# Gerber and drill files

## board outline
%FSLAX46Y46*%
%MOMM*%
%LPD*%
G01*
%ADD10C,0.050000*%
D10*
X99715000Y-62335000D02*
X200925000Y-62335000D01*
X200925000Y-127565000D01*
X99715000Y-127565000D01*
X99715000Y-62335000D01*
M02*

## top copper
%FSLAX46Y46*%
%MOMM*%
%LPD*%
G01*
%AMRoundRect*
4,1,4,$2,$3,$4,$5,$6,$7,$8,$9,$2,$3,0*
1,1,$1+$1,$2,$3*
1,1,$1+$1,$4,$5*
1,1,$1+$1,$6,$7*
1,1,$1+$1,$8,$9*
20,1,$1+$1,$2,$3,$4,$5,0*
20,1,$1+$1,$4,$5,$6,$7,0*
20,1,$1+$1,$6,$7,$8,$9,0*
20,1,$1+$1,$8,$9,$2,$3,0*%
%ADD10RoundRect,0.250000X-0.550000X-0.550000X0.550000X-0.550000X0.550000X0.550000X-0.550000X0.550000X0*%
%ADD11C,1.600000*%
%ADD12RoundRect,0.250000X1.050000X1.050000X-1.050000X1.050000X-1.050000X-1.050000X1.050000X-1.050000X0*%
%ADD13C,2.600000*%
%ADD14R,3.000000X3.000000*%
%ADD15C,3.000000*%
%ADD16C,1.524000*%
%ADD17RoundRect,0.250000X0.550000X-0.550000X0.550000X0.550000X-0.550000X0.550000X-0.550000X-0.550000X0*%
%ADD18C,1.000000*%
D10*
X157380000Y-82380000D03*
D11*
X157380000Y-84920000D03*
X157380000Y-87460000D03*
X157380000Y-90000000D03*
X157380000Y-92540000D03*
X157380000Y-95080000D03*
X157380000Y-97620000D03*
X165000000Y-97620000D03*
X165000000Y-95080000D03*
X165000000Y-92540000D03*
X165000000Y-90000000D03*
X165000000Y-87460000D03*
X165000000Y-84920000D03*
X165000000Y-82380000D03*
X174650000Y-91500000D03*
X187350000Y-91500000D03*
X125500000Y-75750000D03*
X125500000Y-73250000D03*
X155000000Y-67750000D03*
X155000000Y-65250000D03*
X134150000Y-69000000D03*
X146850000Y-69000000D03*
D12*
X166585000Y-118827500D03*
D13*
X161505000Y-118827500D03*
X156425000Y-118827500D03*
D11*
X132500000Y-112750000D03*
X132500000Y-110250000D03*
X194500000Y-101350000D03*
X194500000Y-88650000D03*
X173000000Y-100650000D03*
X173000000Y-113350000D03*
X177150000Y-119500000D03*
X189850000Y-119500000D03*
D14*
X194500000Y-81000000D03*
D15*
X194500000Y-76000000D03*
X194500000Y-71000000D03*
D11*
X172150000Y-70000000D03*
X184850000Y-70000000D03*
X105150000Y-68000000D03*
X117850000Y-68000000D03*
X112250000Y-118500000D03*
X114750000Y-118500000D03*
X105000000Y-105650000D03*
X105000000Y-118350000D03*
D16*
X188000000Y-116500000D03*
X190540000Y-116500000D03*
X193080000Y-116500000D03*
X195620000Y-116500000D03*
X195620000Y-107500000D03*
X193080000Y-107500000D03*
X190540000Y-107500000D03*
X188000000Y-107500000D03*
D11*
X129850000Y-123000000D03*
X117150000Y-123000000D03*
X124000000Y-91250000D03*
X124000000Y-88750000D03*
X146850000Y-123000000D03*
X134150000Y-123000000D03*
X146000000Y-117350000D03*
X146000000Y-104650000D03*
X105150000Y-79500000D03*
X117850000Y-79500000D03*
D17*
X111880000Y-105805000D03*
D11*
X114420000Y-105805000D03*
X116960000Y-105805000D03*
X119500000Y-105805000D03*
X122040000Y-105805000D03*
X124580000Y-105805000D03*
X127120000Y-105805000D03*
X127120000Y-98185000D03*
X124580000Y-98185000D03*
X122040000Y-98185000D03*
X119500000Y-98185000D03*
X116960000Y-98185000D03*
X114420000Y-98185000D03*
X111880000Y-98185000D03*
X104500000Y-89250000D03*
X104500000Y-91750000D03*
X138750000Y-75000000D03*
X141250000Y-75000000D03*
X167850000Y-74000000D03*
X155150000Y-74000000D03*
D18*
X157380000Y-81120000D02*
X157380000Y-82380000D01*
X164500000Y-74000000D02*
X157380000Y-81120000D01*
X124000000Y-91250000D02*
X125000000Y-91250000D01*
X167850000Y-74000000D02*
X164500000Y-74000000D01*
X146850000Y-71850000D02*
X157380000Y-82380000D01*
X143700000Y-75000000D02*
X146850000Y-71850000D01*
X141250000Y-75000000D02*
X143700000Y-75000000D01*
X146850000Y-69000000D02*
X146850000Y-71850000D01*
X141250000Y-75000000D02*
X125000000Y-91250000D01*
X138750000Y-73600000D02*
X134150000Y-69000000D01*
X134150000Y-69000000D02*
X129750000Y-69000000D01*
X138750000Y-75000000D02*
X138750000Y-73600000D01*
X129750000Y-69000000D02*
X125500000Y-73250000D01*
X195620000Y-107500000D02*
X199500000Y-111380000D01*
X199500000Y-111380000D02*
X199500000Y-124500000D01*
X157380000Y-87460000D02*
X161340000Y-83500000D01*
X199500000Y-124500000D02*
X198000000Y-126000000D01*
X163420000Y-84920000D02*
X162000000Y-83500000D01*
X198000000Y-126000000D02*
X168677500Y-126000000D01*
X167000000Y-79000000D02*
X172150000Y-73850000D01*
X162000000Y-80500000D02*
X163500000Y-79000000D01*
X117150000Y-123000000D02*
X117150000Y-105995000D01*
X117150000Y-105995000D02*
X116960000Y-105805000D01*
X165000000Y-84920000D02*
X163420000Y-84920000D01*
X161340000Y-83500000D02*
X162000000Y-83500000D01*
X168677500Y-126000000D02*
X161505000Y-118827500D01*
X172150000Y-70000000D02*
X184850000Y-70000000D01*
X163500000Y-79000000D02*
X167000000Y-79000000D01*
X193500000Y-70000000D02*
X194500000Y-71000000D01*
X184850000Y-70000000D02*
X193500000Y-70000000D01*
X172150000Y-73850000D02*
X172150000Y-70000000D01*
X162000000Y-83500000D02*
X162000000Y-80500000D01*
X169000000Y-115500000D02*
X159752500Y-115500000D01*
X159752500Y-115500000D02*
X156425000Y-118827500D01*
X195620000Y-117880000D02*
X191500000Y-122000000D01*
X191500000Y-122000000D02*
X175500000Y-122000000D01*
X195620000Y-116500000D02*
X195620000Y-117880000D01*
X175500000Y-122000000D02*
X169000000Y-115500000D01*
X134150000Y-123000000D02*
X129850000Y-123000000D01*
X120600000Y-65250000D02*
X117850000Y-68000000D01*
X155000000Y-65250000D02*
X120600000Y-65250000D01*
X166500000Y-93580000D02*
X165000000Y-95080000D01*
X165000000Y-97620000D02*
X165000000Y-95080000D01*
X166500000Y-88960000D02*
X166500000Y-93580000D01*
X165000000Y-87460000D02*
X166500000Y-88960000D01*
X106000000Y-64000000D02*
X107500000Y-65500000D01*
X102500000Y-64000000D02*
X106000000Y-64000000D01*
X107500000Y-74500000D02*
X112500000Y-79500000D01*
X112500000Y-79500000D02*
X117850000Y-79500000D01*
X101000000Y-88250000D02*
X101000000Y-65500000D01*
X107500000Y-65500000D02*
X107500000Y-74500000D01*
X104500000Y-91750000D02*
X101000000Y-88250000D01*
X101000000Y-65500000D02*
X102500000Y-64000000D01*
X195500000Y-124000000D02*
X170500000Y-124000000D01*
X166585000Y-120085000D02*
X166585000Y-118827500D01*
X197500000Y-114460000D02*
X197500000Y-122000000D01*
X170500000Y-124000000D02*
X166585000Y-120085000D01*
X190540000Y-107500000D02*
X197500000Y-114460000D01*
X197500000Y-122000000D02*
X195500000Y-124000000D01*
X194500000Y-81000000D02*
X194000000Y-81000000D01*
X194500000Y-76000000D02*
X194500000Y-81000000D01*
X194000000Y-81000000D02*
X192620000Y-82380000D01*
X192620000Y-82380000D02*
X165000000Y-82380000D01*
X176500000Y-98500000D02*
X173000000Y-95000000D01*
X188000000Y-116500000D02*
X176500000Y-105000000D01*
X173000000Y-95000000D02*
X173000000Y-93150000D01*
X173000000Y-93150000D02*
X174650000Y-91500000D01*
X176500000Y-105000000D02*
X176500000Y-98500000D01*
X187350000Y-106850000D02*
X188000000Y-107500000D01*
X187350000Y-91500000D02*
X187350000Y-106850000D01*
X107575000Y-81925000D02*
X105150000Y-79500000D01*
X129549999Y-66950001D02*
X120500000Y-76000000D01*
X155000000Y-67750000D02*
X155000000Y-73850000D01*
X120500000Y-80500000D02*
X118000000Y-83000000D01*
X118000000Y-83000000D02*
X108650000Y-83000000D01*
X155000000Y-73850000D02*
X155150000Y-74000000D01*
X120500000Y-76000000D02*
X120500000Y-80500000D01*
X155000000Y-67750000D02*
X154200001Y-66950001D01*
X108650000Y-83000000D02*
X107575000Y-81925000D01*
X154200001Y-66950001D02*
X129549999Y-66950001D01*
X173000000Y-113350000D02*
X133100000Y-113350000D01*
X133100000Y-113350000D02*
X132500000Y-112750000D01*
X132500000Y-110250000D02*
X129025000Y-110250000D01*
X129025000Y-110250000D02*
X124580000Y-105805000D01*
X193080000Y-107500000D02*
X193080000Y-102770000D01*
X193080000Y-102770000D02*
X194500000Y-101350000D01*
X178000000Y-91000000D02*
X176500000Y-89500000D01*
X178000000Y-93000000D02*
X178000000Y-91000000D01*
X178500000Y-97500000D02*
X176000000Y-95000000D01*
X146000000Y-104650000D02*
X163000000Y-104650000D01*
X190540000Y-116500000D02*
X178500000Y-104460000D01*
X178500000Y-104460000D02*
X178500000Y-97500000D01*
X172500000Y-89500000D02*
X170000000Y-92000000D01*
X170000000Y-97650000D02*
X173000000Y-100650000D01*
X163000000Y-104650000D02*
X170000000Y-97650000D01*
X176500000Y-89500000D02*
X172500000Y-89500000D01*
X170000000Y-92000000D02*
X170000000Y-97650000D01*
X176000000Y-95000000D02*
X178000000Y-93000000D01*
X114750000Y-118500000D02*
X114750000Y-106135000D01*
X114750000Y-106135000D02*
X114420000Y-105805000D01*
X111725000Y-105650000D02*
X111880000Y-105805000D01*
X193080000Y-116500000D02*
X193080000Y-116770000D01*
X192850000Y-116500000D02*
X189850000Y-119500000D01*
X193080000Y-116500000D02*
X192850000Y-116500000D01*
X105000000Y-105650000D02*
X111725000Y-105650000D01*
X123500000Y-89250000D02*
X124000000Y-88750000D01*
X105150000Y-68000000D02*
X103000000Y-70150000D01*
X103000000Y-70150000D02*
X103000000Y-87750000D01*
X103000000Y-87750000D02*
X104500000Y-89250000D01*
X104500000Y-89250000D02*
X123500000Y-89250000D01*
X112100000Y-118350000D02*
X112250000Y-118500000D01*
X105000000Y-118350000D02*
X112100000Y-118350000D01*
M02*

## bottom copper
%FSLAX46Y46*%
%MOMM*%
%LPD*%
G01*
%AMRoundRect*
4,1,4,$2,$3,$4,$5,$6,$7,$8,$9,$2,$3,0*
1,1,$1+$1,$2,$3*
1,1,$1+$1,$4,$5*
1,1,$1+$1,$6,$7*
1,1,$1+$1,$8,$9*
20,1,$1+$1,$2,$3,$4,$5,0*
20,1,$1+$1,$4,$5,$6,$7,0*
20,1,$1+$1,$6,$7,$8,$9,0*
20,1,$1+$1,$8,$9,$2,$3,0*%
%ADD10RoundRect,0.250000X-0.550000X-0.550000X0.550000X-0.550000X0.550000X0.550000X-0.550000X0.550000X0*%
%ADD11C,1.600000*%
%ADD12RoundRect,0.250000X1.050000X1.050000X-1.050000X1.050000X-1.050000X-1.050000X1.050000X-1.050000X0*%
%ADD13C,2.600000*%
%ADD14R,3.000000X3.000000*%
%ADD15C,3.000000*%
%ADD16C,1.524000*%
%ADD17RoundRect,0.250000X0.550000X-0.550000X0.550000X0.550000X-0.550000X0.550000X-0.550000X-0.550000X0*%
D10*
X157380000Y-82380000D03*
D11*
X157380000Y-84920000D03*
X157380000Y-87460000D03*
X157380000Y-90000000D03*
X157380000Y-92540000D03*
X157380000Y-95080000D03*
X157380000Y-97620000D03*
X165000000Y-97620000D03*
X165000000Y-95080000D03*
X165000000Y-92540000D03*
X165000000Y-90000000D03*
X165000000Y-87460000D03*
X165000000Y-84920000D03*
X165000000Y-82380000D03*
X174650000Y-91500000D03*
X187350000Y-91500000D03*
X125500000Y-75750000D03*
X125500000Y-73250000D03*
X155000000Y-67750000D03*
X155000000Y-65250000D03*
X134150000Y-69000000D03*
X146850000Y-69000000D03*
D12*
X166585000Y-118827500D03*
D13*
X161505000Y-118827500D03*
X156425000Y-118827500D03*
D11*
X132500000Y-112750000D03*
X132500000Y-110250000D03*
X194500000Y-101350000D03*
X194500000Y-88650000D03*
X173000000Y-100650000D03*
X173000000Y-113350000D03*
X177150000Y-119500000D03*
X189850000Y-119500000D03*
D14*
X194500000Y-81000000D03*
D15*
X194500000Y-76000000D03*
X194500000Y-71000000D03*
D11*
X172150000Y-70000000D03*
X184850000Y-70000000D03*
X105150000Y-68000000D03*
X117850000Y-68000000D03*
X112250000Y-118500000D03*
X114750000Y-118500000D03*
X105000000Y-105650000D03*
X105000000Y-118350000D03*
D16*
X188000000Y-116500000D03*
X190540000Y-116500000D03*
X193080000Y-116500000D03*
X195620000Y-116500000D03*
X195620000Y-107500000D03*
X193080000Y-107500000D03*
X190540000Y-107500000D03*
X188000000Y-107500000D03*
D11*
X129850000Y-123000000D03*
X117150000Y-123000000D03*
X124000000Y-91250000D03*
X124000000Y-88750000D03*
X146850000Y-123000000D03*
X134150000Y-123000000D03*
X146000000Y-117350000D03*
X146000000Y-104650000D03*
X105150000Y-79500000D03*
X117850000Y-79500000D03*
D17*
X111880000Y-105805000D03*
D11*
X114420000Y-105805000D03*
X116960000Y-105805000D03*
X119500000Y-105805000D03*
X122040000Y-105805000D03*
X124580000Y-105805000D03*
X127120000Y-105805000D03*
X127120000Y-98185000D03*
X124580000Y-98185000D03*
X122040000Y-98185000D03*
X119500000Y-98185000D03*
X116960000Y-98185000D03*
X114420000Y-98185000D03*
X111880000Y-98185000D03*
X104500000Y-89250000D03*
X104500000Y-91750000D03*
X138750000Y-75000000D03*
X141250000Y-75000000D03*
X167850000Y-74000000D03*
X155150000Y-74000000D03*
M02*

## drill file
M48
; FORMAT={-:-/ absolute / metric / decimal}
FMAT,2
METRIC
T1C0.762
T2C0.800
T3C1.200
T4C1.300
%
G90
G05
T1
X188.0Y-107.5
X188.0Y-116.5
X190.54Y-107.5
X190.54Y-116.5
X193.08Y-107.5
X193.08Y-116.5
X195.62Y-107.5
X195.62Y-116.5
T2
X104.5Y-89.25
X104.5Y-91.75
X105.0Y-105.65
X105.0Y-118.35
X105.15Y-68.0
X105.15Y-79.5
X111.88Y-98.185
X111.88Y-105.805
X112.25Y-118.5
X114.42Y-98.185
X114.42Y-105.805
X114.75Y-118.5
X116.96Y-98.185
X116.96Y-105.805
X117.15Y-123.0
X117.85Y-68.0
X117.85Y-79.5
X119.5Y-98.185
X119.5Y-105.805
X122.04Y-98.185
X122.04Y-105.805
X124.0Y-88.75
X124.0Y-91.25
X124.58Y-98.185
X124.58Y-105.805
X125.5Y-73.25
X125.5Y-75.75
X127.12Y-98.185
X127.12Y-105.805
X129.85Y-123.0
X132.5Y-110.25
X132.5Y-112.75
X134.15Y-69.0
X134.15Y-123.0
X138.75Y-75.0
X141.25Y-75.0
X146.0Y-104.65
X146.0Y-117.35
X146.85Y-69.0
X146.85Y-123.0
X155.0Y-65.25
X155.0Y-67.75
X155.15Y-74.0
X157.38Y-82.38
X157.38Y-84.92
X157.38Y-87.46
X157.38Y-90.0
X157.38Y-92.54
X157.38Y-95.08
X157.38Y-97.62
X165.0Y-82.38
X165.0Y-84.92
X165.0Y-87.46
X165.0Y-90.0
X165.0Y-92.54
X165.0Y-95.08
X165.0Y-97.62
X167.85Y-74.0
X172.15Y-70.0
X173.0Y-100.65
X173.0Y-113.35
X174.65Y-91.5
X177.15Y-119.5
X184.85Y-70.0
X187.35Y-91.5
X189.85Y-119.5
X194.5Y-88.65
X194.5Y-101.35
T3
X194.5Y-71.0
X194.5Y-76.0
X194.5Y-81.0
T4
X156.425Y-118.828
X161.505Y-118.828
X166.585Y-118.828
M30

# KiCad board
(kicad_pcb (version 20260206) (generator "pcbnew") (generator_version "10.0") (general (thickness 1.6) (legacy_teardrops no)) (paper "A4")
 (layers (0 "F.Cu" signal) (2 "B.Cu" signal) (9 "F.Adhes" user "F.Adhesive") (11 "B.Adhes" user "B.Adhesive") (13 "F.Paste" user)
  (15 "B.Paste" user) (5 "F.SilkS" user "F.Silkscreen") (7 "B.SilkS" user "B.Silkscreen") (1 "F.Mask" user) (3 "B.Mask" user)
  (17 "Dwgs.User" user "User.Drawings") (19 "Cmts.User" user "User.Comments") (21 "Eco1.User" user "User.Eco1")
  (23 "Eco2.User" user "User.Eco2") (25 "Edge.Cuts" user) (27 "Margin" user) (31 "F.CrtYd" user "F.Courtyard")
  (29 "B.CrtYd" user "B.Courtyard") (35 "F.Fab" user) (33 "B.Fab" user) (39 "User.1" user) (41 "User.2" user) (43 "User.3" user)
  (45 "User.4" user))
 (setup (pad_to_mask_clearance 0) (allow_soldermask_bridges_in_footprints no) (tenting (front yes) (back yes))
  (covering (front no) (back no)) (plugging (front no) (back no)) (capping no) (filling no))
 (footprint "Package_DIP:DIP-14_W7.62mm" (layer "F.Cu") (at 157.38 82.38)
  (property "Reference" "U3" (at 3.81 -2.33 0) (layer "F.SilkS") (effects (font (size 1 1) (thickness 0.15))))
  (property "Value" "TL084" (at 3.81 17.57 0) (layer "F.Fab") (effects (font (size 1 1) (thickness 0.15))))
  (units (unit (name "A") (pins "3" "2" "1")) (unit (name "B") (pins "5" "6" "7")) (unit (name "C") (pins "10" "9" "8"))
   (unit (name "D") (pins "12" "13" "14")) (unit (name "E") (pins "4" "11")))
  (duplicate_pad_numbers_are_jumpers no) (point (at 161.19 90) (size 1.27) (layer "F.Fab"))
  (pad "1" thru_hole roundrect (at 0 0) (size 1.6 1.6) (drill 0.8) (layers "*.Cu" "*.Mask") (remove_unused_layers no)
   (roundrect_rratio 0.15625) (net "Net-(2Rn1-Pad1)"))
  (pad "2" thru_hole circle (at 0 2.54) (size 1.6 1.6) (drill 0.8) (layers "*.Cu" "*.Mask") (remove_unused_layers no) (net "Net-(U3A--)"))
  (pad "3" thru_hole circle (at 0 5.08) (size 1.6 1.6) (drill 0.8) (layers "*.Cu" "*.Mask") (remove_unused_layers no) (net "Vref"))
  (pad "4" thru_hole circle (at 0 7.62) (size 1.6 1.6) (drill 0.8) (layers "*.Cu" "*.Mask") (remove_unused_layers no) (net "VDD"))
  (pad "5" thru_hole circle (at 0 10.16) (size 1.6 1.6) (drill 0.8) (layers "*.Cu" "*.Mask") (remove_unused_layers no) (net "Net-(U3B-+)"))
  (pad "6" thru_hole circle (at 0 12.7) (size 1.6 1.6) (drill 0.8) (layers "*.Cu" "*.Mask") (remove_unused_layers no) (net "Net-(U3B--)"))
  (pad "7" thru_hole circle (at 0 15.24) (size 1.6 1.6) (drill 0.8) (layers "*.Cu" "*.Mask") (remove_unused_layers no) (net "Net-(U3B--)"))
  (pad "8" thru_hole circle (at 7.62 15.24) (size 1.6 1.6) (drill 0.8) (layers "*.Cu" "*.Mask") (remove_unused_layers no)
   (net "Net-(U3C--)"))
  (pad "9" thru_hole circle (at 7.62 12.7) (size 1.6 1.6) (drill 0.8) (layers "*.Cu" "*.Mask") (remove_unused_layers no) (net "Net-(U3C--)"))
  (pad "10" thru_hole circle (at 7.62 10.16) (size 1.6 1.6) (drill 0.8) (layers "*.Cu" "*.Mask") (remove_unused_layers no)
   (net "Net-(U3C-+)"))
  (pad "11" thru_hole circle (at 7.62 7.62) (size 1.6 1.6) (drill 0.8) (layers "*.Cu" "*.Mask") (remove_unused_layers no) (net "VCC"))
  (pad "12" thru_hole circle (at 7.62 5.08) (size 1.6 1.6) (drill 0.8) (layers "*.Cu" "*.Mask") (remove_unused_layers no)
   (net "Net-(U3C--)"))
  (pad "13" thru_hole circle (at 7.62 2.54) (size 1.6 1.6) (drill 0.8) (layers "*.Cu" "*.Mask") (remove_unused_layers no) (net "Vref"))
  (pad "14" thru_hole circle (at 7.62 0) (size 1.6 1.6) (drill 0.8) (layers "*.Cu" "*.Mask") (remove_unused_layers no) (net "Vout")))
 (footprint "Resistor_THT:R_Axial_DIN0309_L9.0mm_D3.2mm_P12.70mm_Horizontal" (layer "F.Cu") (at 174.65 91.5)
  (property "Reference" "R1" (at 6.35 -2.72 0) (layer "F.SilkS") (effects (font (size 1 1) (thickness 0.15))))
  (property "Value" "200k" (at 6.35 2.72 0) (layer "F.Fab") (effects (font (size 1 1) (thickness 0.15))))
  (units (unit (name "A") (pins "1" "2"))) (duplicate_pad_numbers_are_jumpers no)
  (pad "1" thru_hole circle (at 0 0) (size 1.6 1.6) (drill 0.8) (layers "*.Cu" "*.Mask") (remove_unused_layers no) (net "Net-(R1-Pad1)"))
  (pad "2" thru_hole circle (at 12.7 0) (size 1.6 1.6) (drill 0.8) (layers "*.Cu" "*.Mask") (remove_unused_layers no) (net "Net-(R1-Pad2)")))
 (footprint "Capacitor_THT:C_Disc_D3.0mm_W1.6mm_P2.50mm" (layer "F.Cu") (at 125.5 75.75 90)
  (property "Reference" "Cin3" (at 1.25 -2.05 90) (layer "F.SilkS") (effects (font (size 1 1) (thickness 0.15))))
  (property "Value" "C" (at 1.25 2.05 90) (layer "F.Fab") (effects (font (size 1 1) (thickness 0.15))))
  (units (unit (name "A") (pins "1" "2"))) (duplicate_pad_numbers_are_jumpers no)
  (pad "1" thru_hole circle (at 0 0 90) (size 1.6 1.6) (drill 0.8) (layers "*.Cu" "*.Mask") (remove_unused_layers no)
   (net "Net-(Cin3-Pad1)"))
  (pad "2" thru_hole circle (at 2.5 0 90) (size 1.6 1.6) (drill 0.8) (layers "*.Cu" "*.Mask") (remove_unused_layers no) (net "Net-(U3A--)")))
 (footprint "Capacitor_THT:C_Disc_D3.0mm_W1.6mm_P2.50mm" (layer "F.Cu") (at 155 67.75 90)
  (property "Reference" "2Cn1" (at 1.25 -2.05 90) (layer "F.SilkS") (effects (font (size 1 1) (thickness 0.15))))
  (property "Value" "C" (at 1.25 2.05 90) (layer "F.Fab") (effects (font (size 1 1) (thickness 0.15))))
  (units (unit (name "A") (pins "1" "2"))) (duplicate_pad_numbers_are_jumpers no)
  (pad "1" thru_hole circle (at 0 0 90) (size 1.6 1.6) (drill 0.8) (layers "*.Cu" "*.Mask") (remove_unused_layers no)
   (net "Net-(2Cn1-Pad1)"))
  (pad "2" thru_hole circle (at 2.5 0 90) (size 1.6 1.6) (drill 0.8) (layers "*.Cu" "*.Mask") (remove_unused_layers no) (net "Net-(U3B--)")))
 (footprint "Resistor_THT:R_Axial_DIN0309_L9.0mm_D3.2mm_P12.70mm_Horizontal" (layer "F.Cu") (at 134.15 69)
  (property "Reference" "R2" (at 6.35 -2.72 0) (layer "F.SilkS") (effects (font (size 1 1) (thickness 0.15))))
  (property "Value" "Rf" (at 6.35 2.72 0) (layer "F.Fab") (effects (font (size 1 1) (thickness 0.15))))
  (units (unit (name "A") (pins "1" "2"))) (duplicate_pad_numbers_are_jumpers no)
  (pad "1" thru_hole circle (at 0 0) (size 1.6 1.6) (drill 0.8) (layers "*.Cu" "*.Mask") (remove_unused_layers no) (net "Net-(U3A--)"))
  (pad "2" thru_hole circle (at 12.7 0) (size 1.6 1.6) (drill 0.8) (layers "*.Cu" "*.Mask") (remove_unused_layers no)
   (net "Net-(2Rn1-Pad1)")))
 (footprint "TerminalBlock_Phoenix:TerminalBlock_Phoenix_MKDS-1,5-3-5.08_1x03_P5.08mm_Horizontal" (layer "F.Cu") (at 166.585 118.8275 180)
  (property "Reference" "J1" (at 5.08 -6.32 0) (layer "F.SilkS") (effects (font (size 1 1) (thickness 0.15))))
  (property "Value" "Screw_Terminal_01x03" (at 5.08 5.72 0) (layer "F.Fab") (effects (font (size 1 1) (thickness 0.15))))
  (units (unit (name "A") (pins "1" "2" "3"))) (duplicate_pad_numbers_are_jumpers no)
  (pad "1" thru_hole roundrect (at 0 0 180) (size 2.6 2.6) (drill 1.3) (layers "*.Cu" "*.Mask") (remove_unused_layers no)
   (roundrect_rratio 0.096154) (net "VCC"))
  (pad "2" thru_hole circle (at 5.08 0 180) (size 2.6 2.6) (drill 1.3) (layers "*.Cu" "*.Mask") (remove_unused_layers no) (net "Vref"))
  (pad "3" thru_hole circle (at 10.16 0 180) (size 2.6 2.6) (drill 1.3) (layers "*.Cu" "*.Mask") (remove_unused_layers no) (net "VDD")))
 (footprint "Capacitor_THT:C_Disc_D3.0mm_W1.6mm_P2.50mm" (layer "F.Cu") (at 132.5 112.75 90)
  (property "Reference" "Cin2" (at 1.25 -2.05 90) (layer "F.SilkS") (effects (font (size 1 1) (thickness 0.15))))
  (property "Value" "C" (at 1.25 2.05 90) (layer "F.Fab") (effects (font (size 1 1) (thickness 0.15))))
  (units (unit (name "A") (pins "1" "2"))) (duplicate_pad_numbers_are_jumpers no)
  (pad "1" thru_hole circle (at 0 0 90) (size 1.6 1.6) (drill 0.8) (layers "*.Cu" "*.Mask") (remove_unused_layers no)
   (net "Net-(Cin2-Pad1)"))
  (pad "2" thru_hole circle (at 2.5 0 90) (size 1.6 1.6) (drill 0.8) (layers "*.Cu" "*.Mask") (remove_unused_layers no) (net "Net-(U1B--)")))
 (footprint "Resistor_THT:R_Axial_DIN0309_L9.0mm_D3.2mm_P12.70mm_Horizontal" (layer "F.Cu") (at 194.5 101.35 90)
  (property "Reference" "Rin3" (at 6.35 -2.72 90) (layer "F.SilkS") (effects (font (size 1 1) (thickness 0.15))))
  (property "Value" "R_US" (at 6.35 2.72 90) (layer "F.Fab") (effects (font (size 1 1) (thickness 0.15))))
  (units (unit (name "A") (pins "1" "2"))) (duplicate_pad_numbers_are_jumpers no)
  (pad "1" thru_hole circle (at 0 0 90) (size 1.6 1.6) (drill 0.8) (layers "*.Cu" "*.Mask") (remove_unused_layers no) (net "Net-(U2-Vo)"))
  (pad "2" thru_hole circle (at 12.7 0 90) (size 1.6 1.6) (drill 0.8) (layers "*.Cu" "*.Mask") (remove_unused_layers no)
   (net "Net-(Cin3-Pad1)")))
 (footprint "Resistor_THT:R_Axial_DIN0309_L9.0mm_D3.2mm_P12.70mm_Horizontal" (layer "F.Cu") (at 173 100.65 -90)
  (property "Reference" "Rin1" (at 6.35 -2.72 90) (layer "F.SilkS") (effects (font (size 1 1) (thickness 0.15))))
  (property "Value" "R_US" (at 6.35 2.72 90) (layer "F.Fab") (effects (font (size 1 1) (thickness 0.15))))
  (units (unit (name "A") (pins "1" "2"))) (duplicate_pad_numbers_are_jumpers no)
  (pad "1" thru_hole circle (at 0 0 270) (size 1.6 1.6) (drill 0.8) (layers "*.Cu" "*.Mask") (remove_unused_layers no) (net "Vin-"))
  (pad "2" thru_hole circle (at 12.7 0 270) (size 1.6 1.6) (drill 0.8) (layers "*.Cu" "*.Mask") (remove_unused_layers no)
   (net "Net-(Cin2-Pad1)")))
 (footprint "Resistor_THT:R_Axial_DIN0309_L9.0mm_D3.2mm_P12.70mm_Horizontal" (layer "F.Cu") (at 177.15 119.5)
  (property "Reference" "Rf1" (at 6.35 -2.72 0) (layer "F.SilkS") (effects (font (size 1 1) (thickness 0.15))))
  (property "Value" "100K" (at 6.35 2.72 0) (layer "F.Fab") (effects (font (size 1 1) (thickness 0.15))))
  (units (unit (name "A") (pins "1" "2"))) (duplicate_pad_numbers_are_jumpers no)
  (pad "1" thru_hole circle (at 0 0) (size 1.6 1.6) (drill 0.8) (layers "*.Cu" "*.Mask") (remove_unused_layers no) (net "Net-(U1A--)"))
  (pad "2" thru_hole circle (at 12.7 0) (size 1.6 1.6) (drill 0.8) (layers "*.Cu" "*.Mask") (remove_unused_layers no) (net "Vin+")))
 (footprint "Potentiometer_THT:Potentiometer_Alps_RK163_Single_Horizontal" (layer "F.Cu") (at 194.5 81 180)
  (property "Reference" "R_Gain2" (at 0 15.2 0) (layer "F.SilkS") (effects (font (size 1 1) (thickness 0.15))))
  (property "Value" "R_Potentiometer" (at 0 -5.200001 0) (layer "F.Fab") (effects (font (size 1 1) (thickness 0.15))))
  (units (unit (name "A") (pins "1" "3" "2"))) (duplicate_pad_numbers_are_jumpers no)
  (pad "1" thru_hole rect (at 0 0) (size 3 3) (drill 1.2) (layers "*.Cu" "*.Mask") (remove_unused_layers no) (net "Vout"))
  (pad "2" thru_hole circle (at 0 5) (size 3 3) (drill 1.2) (layers "*.Cu" "*.Mask") (remove_unused_layers no) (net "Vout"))
  (pad "3" thru_hole circle (at 0 10) (size 3 3) (drill 1.2) (layers "*.Cu" "*.Mask") (remove_unused_layers no) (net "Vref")))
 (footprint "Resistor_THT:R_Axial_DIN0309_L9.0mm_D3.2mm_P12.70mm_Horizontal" (layer "F.Cu") (at 172.15 70)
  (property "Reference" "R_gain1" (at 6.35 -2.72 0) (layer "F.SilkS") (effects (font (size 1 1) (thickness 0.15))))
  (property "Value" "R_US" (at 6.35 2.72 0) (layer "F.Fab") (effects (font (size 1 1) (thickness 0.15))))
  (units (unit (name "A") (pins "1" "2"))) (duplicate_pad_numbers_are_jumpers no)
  (pad "1" thru_hole circle (at 0 0) (size 1.6 1.6) (drill 0.8) (layers "*.Cu" "*.Mask") (remove_unused_layers no) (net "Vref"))
  (pad "2" thru_hole circle (at 12.7 0) (size 1.6 1.6) (drill 0.8) (layers "*.Cu" "*.Mask") (remove_unused_layers no) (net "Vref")))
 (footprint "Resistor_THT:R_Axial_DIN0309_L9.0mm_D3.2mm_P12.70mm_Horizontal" (layer "F.Cu") (at 105.15 68)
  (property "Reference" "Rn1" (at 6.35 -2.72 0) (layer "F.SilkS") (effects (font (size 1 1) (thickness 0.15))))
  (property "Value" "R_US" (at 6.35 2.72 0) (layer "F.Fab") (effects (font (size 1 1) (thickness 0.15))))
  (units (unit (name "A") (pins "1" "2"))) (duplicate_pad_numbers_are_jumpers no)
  (pad "1" thru_hole circle (at 0 0) (size 1.6 1.6) (drill 0.8) (layers "*.Cu" "*.Mask") (remove_unused_layers no) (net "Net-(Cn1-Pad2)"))
  (pad "2" thru_hole circle (at 12.7 0) (size 1.6 1.6) (drill 0.8) (layers "*.Cu" "*.Mask") (remove_unused_layers no) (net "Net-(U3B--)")))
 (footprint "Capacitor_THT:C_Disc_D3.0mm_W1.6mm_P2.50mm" (layer "F.Cu") (at 112.25 118.5)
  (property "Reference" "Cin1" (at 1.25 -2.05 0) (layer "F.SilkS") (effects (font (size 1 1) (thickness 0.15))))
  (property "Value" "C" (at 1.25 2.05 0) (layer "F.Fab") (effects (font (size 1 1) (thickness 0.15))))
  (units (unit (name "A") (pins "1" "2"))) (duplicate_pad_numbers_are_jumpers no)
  (pad "1" thru_hole circle (at 0 0) (size 1.6 1.6) (drill 0.8) (layers "*.Cu" "*.Mask") (remove_unused_layers no) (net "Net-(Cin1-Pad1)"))
  (pad "2" thru_hole circle (at 2.5 0) (size 1.6 1.6) (drill 0.8) (layers "*.Cu" "*.Mask") (remove_unused_layers no) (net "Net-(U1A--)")))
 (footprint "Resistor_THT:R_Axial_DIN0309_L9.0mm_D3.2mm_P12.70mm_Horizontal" (layer "F.Cu") (at 105 105.65 -90)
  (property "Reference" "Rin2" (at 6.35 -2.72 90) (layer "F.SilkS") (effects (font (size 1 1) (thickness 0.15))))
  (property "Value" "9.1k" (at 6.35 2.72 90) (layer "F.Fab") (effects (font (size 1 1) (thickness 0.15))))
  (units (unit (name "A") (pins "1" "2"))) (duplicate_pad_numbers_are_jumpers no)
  (pad "1" thru_hole circle (at 0 0 270) (size 1.6 1.6) (drill 0.8) (layers "*.Cu" "*.Mask") (remove_unused_layers no) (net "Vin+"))
  (pad "2" thru_hole circle (at 12.7 0 270) (size 1.6 1.6) (drill 0.8) (layers "*.Cu" "*.Mask") (remove_unused_layers no)
   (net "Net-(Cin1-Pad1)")))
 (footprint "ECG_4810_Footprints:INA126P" (layer "F.Cu") (at 192 112 90)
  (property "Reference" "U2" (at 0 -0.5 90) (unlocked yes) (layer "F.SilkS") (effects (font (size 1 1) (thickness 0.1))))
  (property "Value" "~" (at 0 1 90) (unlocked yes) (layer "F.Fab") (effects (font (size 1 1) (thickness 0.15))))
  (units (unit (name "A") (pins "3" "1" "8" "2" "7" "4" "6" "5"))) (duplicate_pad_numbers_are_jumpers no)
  (pad "1" thru_hole circle (at -4.5 -4) (size 1.524 1.524) (drill 0.762) (layers "*.Cu" "*.Mask") (remove_unused_layers no)
   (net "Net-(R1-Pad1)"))
  (pad "2" thru_hole circle (at -4.5 -1.46) (size 1.524 1.524) (drill 0.762) (layers "*.Cu" "*.Mask") (remove_unused_layers no) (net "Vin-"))
  (pad "3" thru_hole circle (at -4.5 1.08) (size 1.524 1.524) (drill 0.762) (layers "*.Cu" "*.Mask") (remove_unused_layers no) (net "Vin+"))
  (pad "4" thru_hole circle (at -4.5 3.62) (size 1.524 1.524) (drill 0.762) (layers "*.Cu" "*.Mask") (remove_unused_layers no) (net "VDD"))
  (pad "5" thru_hole circle (at 4.5 3.62 180) (size 1.524 1.524) (drill 0.762) (layers "*.Cu" "*.Mask") (remove_unused_layers no)
   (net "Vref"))
  (pad "6" thru_hole circle (at 4.5 1.08 180) (size 1.524 1.524) (drill 0.762) (layers "*.Cu" "*.Mask") (remove_unused_layers no)
   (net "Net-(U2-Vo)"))
  (pad "7" thru_hole circle (at 4.5 -1.46 180) (size 1.524 1.524) (drill 0.762) (layers "*.Cu" "*.Mask") (remove_unused_layers no)
   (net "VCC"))
  (pad "8" thru_hole circle (at 4.5 -4 180) (size 1.524 1.524) (drill 0.762) (layers "*.Cu" "*.Mask") (remove_unused_layers no)
   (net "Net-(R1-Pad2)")))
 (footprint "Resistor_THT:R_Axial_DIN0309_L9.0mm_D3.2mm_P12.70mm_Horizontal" (layer "F.Cu") (at 129.85 123 180)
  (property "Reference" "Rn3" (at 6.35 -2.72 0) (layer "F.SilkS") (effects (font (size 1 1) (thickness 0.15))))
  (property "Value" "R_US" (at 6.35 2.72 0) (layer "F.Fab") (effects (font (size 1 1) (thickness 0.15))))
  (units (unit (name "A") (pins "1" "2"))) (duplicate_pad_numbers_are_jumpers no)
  (pad "1" thru_hole circle (at 0 0 180) (size 1.6 1.6) (drill 0.8) (layers "*.Cu" "*.Mask") (remove_unused_layers no) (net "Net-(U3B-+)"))
  (pad "2" thru_hole circle (at 12.7 0 180) (size 1.6 1.6) (drill 0.8) (layers "*.Cu" "*.Mask") (remove_unused_layers no) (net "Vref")))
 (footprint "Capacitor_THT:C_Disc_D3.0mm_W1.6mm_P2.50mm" (layer "F.Cu") (at 124 91.25 90)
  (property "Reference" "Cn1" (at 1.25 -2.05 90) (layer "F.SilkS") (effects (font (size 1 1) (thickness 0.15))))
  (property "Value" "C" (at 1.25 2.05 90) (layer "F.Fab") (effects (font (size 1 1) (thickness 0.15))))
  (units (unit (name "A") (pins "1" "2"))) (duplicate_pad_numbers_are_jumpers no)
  (pad "1" thru_hole circle (at 0 0 90) (size 1.6 1.6) (drill 0.8) (layers "*.Cu" "*.Mask") (remove_unused_layers no)
   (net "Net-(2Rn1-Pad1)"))
  (pad "2" thru_hole circle (at 2.5 0 90) (size 1.6 1.6) (drill 0.8) (layers "*.Cu" "*.Mask") (remove_unused_layers no)
   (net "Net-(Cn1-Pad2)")))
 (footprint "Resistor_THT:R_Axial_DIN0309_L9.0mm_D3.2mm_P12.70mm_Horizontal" (layer "F.Cu") (at 146.85 123 180)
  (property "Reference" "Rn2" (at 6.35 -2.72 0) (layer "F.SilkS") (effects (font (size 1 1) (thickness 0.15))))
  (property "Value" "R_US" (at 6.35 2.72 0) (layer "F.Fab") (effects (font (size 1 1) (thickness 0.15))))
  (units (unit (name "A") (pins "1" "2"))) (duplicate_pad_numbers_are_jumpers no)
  (pad "1" thru_hole circle (at 0 0 180) (size 1.6 1.6) (drill 0.8) (layers "*.Cu" "*.Mask") (remove_unused_layers no) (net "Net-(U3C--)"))
  (pad "2" thru_hole circle (at 12.7 0 180) (size 1.6 1.6) (drill 0.8) (layers "*.Cu" "*.Mask") (remove_unused_layers no)
   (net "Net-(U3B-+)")))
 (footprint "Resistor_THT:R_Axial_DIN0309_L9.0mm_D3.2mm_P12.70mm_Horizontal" (layer "F.Cu") (at 146 117.35 90)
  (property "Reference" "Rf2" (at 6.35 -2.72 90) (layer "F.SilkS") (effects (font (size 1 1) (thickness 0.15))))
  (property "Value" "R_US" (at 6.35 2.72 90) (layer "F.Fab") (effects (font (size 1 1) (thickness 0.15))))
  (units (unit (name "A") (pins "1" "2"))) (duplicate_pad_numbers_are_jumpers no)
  (pad "1" thru_hole circle (at 0 0 90) (size 1.6 1.6) (drill 0.8) (layers "*.Cu" "*.Mask") (remove_unused_layers no) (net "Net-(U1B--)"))
  (pad "2" thru_hole circle (at 12.7 0 90) (size 1.6 1.6) (drill 0.8) (layers "*.Cu" "*.Mask") (remove_unused_layers no) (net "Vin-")))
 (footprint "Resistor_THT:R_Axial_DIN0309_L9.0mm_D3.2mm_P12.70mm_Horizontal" (layer "F.Cu") (at 105.15 79.5)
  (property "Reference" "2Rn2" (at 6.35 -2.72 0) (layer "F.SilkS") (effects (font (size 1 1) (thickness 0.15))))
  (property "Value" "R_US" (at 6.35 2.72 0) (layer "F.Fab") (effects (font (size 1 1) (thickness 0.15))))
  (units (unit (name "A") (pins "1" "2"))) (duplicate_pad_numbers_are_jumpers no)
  (pad "1" thru_hole circle (at 0 0) (size 1.6 1.6) (drill 0.8) (layers "*.Cu" "*.Mask") (remove_unused_layers no) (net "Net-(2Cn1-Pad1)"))
  (pad "2" thru_hole circle (at 12.7 0) (size 1.6 1.6) (drill 0.8) (layers "*.Cu" "*.Mask") (remove_unused_layers no) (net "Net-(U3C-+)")))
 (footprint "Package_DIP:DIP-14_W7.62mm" (layer "F.Cu") (at 111.88 105.805 90)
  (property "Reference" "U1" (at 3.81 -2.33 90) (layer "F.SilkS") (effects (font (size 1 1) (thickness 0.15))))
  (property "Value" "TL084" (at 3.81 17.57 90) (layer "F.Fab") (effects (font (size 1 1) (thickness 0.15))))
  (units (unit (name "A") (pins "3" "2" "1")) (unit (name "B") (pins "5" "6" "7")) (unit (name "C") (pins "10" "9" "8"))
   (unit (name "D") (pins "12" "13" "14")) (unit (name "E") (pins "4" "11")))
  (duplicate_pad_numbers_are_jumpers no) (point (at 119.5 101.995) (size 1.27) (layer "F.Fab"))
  (pad "1" thru_hole roundrect (at 0 0 90) (size 1.6 1.6) (drill 0.8) (layers "*.Cu" "*.Mask") (remove_unused_layers no)
   (roundrect_rratio 0.15625) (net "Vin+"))
  (pad "2" thru_hole circle (at 0 2.54 90) (size 1.6 1.6) (drill 0.8) (layers "*.Cu" "*.Mask") (remove_unused_layers no) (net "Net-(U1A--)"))
  (pad "3" thru_hole circle (at 0 5.08 90) (size 1.6 1.6) (drill 0.8) (layers "*.Cu" "*.Mask") (remove_unused_layers no) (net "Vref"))
  (pad "4" thru_hole circle (at 0 7.62 90) (size 1.6 1.6) (drill 0.8) (layers "*.Cu" "*.Mask") (remove_unused_layers no) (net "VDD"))
  (pad "5" thru_hole circle (at 0 10.16 90) (size 1.6 1.6) (drill 0.8) (layers "*.Cu" "*.Mask") (remove_unused_layers no) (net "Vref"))
  (pad "6" thru_hole circle (at 0 12.7 90) (size 1.6 1.6) (drill 0.8) (layers "*.Cu" "*.Mask") (remove_unused_layers no) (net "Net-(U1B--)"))
  (pad "7" thru_hole circle (at 0 15.24 90) (size 1.6 1.6) (drill 0.8) (layers "*.Cu" "*.Mask") (remove_unused_layers no) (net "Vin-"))
  (pad "8" thru_hole circle (at 7.62 15.24 90) (size 1.6 1.6) (drill 0.8) (layers "*.Cu" "*.Mask") (remove_unused_layers no))
  (pad "9" thru_hole circle (at 7.62 12.7 90) (size 1.6 1.6) (drill 0.8) (layers "*.Cu" "*.Mask") (remove_unused_layers no))
  (pad "10" thru_hole circle (at 7.62 10.16 90) (size 1.6 1.6) (drill 0.8) (layers "*.Cu" "*.Mask") (remove_unused_layers no))
  (pad "11" thru_hole circle (at 7.62 7.62 90) (size 1.6 1.6) (drill 0.8) (layers "*.Cu" "*.Mask") (remove_unused_layers no) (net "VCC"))
  (pad "12" thru_hole circle (at 7.62 5.08 90) (size 1.6 1.6) (drill 0.8) (layers "*.Cu" "*.Mask") (remove_unused_layers no))
  (pad "13" thru_hole circle (at 7.62 2.54 90) (size 1.6 1.6) (drill 0.8) (layers "*.Cu" "*.Mask") (remove_unused_layers no))
  (pad "14" thru_hole circle (at 7.62 0 90) (size 1.6 1.6) (drill 0.8) (layers "*.Cu" "*.Mask") (remove_unused_layers no)))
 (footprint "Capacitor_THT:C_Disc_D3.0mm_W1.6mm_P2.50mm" (layer "F.Cu") (at 104.5 89.25 -90)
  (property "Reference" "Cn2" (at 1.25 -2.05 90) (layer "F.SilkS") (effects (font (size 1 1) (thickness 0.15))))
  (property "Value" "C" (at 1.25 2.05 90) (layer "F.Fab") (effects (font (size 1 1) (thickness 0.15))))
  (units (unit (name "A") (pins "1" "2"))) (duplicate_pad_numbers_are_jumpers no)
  (pad "1" thru_hole circle (at 0 0 270) (size 1.6 1.6) (drill 0.8) (layers "*.Cu" "*.Mask") (remove_unused_layers no)
   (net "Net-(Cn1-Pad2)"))
  (pad "2" thru_hole circle (at 2.5 0 270) (size 1.6 1.6) (drill 0.8) (layers "*.Cu" "*.Mask") (remove_unused_layers no) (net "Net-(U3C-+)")))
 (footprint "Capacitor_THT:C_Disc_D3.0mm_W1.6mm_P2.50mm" (layer "F.Cu") (at 138.75 75)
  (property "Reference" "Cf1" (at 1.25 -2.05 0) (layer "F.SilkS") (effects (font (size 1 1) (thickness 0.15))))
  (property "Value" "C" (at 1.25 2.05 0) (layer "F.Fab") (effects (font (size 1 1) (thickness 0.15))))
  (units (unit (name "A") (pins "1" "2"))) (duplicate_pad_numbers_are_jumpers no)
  (pad "1" thru_hole circle (at 0 0) (size 1.6 1.6) (drill 0.8) (layers "*.Cu" "*.Mask") (remove_unused_layers no) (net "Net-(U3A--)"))
  (pad "2" thru_hole circle (at 2.5 0) (size 1.6 1.6) (drill 0.8) (layers "*.Cu" "*.Mask") (remove_unused_layers no) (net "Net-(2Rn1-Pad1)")))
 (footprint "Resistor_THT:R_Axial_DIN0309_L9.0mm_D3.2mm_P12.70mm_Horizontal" (layer "F.Cu") (at 167.85 74 180)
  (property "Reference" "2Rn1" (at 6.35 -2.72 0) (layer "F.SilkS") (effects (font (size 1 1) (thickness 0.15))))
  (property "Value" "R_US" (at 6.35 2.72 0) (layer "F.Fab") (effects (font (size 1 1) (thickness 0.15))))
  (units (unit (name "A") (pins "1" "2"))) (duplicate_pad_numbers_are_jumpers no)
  (pad "1" thru_hole circle (at 0 0 180) (size 1.6 1.6) (drill 0.8) (layers "*.Cu" "*.Mask") (remove_unused_layers no)
   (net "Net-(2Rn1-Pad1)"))
  (pad "2" thru_hole circle (at 12.7 0 180) (size 1.6 1.6) (drill 0.8) (layers "*.Cu" "*.Mask") (remove_unused_layers no)
   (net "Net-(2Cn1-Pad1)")))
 (gr_rect (start 99.715 62.335) (end 200.925 127.565) (stroke (width 0.05) (type solid)) (fill no) (layer "Edge.Cuts"))
 (segment (start 157.38 81.12) (end 157.38 82.38) (width 1) (layer "F.Cu") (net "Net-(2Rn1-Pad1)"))
 (segment (start 164.5 74) (end 157.38 81.12) (width 1) (layer "F.Cu") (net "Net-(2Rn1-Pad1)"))
 (segment (start 124 91.25) (end 125 91.25) (width 1) (layer "F.Cu") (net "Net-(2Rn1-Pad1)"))
 (segment (start 167.85 74) (end 164.5 74) (width 1) (layer "F.Cu") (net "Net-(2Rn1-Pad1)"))
 (segment (start 146.85 71.85) (end 157.38 82.38) (width 1) (layer "F.Cu") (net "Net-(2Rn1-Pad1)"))
 (segment (start 143.7 75) (end 146.85 71.85) (width 1) (layer "F.Cu") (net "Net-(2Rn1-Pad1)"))
 (segment (start 141.25 75) (end 143.7 75) (width 1) (layer "F.Cu") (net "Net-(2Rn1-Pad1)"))
 (segment (start 146.85 69) (end 146.85 71.85) (width 1) (layer "F.Cu") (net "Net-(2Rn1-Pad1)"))
 (segment (start 141.25 75) (end 125 91.25) (width 1) (layer "F.Cu") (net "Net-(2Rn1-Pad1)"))
 (segment (start 138.75 73.6) (end 134.15 69) (width 1) (layer "F.Cu") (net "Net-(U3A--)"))
 (segment (start 134.15 69) (end 129.75 69) (width 1) (layer "F.Cu") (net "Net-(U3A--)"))
 (segment (start 138.75 75) (end 138.75 73.6) (width 1) (layer "F.Cu") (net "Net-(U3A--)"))
 (segment (start 129.75 69) (end 125.5 73.25) (width 1) (layer "F.Cu") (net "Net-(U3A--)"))
 (segment (start 195.62 107.5) (end 199.5 111.38) (width 1) (layer "F.Cu") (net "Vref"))
 (segment (start 199.5 111.38) (end 199.5 124.5) (width 1) (layer "F.Cu") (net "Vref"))
 (segment (start 157.38 87.46) (end 161.34 83.5) (width 1) (layer "F.Cu") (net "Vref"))
 (segment (start 199.5 124.5) (end 198 126) (width 1) (layer "F.Cu") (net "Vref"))
 (segment (start 163.42 84.92) (end 162 83.5) (width 1) (layer "F.Cu") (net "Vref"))
 (segment (start 198 126) (end 168.6775 126) (width 1) (layer "F.Cu") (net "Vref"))
 (segment (start 167 79) (end 172.15 73.85) (width 1) (layer "F.Cu") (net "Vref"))
 (segment (start 162 80.5) (end 163.5 79) (width 1) (layer "F.Cu") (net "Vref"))
 (segment (start 117.15 123) (end 117.15 105.995) (width 1) (layer "F.Cu") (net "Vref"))
 (segment (start 117.15 105.995) (end 116.96 105.805) (width 1) (layer "F.Cu") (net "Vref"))
 (segment (start 165 84.92) (end 163.42 84.92) (width 1) (layer "F.Cu") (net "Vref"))
 (segment (start 161.34 83.5) (end 162 83.5) (width 1) (layer "F.Cu") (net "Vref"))
 (segment (start 168.6775 126) (end 161.505 118.8275) (width 1) (layer "F.Cu") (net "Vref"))
 (segment (start 172.15 70) (end 184.85 70) (width 1) (layer "F.Cu") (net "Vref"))
 (segment (start 163.5 79) (end 167 79) (width 1) (layer "F.Cu") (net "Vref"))
 (segment (start 193.5 70) (end 194.5 71) (width 1) (layer "F.Cu") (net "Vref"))
 (segment (start 184.85 70) (end 193.5 70) (width 1) (layer "F.Cu") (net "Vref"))
 (segment (start 172.15 73.85) (end 172.15 70) (width 1) (layer "F.Cu") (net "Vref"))
 (segment (start 162 83.5) (end 162 80.5) (width 1) (layer "F.Cu") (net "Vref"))
 (segment (start 169 115.5) (end 159.7525 115.5) (width 1) (layer "F.Cu") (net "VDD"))
 (segment (start 159.7525 115.5) (end 156.425 118.8275) (width 1) (layer "F.Cu") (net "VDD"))
 (segment (start 195.62 117.88) (end 191.5 122) (width 1) (layer "F.Cu") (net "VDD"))
 (segment (start 191.5 122) (end 175.5 122) (width 1) (layer "F.Cu") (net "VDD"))
 (segment (start 195.62 116.5) (end 195.62 117.88) (width 1) (layer "F.Cu") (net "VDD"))
 (segment (start 175.5 122) (end 169 115.5) (width 1) (layer "F.Cu") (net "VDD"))
 (segment (start 134.15 123) (end 129.85 123) (width 1) (layer "F.Cu") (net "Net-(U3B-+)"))
 (segment (start 120.6 65.25) (end 117.85 68) (width 1) (layer "F.Cu") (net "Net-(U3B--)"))
 (segment (start 155 65.25) (end 120.6 65.25) (width 1) (layer "F.Cu") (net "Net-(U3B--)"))
 (segment (start 166.5 93.58) (end 165 95.08) (width 1) (layer "F.Cu") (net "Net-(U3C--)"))
 (segment (start 165 97.62) (end 165 95.08) (width 1) (layer "F.Cu") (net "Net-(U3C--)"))
 (segment (start 166.5 88.96) (end 166.5 93.58) (width 1) (layer "F.Cu") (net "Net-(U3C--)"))
 (segment (start 165 87.46) (end 166.5 88.96) (width 1) (layer "F.Cu") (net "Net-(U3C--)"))
 (segment (start 106 64) (end 107.5 65.5) (width 1) (layer "F.Cu") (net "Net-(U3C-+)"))
 (segment (start 102.5 64) (end 106 64) (width 1) (layer "F.Cu") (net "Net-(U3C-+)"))
 (segment (start 107.5 74.5) (end 112.5 79.5) (width 1) (layer "F.Cu") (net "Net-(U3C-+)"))
 (segment (start 112.5 79.5) (end 117.85 79.5) (width 1) (layer "F.Cu") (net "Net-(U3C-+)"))
 (segment (start 101 88.25) (end 101 65.5) (width 1) (layer "F.Cu") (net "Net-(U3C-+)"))
 (segment (start 107.5 65.5) (end 107.5 74.5) (width 1) (layer "F.Cu") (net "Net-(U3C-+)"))
 (segment (start 104.5 91.75) (end 101 88.25) (width 1) (layer "F.Cu") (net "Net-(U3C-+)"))
 (segment (start 101 65.5) (end 102.5 64) (width 1) (layer "F.Cu") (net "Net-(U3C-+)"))
 (segment (start 195.5 124) (end 170.5 124) (width 1) (layer "F.Cu") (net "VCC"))
 (segment (start 166.585 120.085) (end 166.585 118.8275) (width 1) (layer "F.Cu") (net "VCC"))
 (segment (start 197.5 114.46) (end 197.5 122) (width 1) (layer "F.Cu") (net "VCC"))
 (segment (start 170.5 124) (end 166.585 120.085) (width 1) (layer "F.Cu") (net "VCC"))
 (segment (start 190.54 107.5) (end 197.5 114.46) (width 1) (layer "F.Cu") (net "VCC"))
 (segment (start 197.5 122) (end 195.5 124) (width 1) (layer "F.Cu") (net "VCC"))
 (segment (start 194.5 81) (end 194 81) (width 1) (layer "F.Cu") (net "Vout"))
 (segment (start 194.5 76) (end 194.5 81) (width 1) (layer "F.Cu") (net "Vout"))
 (segment (start 194 81) (end 192.62 82.38) (width 1) (layer "F.Cu") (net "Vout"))
 (segment (start 192.62 82.38) (end 165 82.38) (width 1) (layer "F.Cu") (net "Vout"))
 (segment (start 176.5 98.5) (end 173 95) (width 1) (layer "F.Cu") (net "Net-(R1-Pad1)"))
 (segment (start 188 116.5) (end 176.5 105) (width 1) (layer "F.Cu") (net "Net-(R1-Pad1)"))
 (segment (start 173 95) (end 173 93.15) (width 1) (layer "F.Cu") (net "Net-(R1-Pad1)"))
 (segment (start 173 93.15) (end 174.65 91.5) (width 1) (layer "F.Cu") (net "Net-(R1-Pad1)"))
 (segment (start 176.5 105) (end 176.5 98.5) (width 1) (layer "F.Cu") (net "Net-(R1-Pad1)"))
 (segment (start 187.35 106.85) (end 188 107.5) (width 1) (layer "F.Cu") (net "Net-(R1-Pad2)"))
 (segment (start 187.35 91.5) (end 187.35 106.85) (width 1) (layer "F.Cu") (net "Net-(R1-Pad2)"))
 (segment (start 107.575 81.925) (end 105.15 79.5) (width 1) (layer "F.Cu") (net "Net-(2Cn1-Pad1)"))
 (segment (start 129.549999 66.950001) (end 120.5 76) (width 1) (layer "F.Cu") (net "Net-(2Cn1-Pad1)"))
 (segment (start 155 67.75) (end 155 73.85) (width 1) (layer "F.Cu") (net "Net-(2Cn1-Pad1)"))
 (segment (start 120.5 80.5) (end 118 83) (width 1) (layer "F.Cu") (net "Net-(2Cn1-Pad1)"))
 (segment (start 118 83) (end 108.65 83) (width 1) (layer "F.Cu") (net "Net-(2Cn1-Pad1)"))
 (segment (start 155 73.85) (end 155.15 74) (width 1) (layer "F.Cu") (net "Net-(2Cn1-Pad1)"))
 (segment (start 120.5 76) (end 120.5 80.5) (width 1) (layer "F.Cu") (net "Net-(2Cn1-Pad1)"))
 (segment (start 155 67.75) (end 154.200001 66.950001) (width 1) (layer "F.Cu") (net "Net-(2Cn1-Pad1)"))
 (segment (start 108.65 83) (end 107.575 81.925) (width 1) (layer "F.Cu") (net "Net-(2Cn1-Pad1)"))
 (segment (start 154.200001 66.950001) (end 129.549999 66.950001) (width 1) (layer "F.Cu") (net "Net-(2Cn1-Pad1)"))
 (segment (start 173 113.35) (end 133.1 113.35) (width 1) (layer "F.Cu") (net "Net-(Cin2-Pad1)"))
 (segment (start 133.1 113.35) (end 132.5 112.75) (width 1) (layer "F.Cu") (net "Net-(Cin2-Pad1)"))
 (segment (start 132.5 110.25) (end 129.025 110.25) (width 1) (layer "F.Cu") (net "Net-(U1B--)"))
 (segment (start 129.025 110.25) (end 124.58 105.805) (width 1) (layer "F.Cu") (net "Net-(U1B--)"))
 (segment (start 193.08 107.5) (end 193.08 102.77) (width 1) (layer "F.Cu") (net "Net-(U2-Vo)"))
 (segment (start 193.08 102.77) (end 194.5 101.35) (width 1) (layer "F.Cu") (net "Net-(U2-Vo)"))
 (segment (start 178 91) (end 176.5 89.5) (width 1) (layer "F.Cu") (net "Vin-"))
 (segment (start 178 93) (end 178 91) (width 1) (layer "F.Cu") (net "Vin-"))
 (segment (start 178.5 97.5) (end 176 95) (width 1) (layer "F.Cu") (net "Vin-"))
 (segment (start 146 104.65) (end 163 104.65) (width 1) (layer "F.Cu") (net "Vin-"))
 (segment (start 190.54 116.5) (end 178.5 104.46) (width 1) (layer "F.Cu") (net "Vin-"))
 (segment (start 178.5 104.46) (end 178.5 97.5) (width 1) (layer "F.Cu") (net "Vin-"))
 (segment (start 172.5 89.5) (end 170 92) (width 1) (layer "F.Cu") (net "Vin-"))
 (segment (start 170 97.65) (end 173 100.65) (width 1) (layer "F.Cu") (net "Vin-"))
 (segment (start 163 104.65) (end 170 97.65) (width 1) (layer "F.Cu") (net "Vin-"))
 (segment (start 176.5 89.5) (end 172.5 89.5) (width 1) (layer "F.Cu") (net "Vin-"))
 (segment (start 170 92) (end 170 97.65) (width 1) (layer "F.Cu") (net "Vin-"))
 (segment (start 176 95) (end 178 93) (width 1) (layer "F.Cu") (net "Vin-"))
 (segment (start 114.75 118.5) (end 114.75 106.135) (width 1) (layer "F.Cu") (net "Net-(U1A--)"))
 (segment (start 114.75 106.135) (end 114.42 105.805) (width 1) (layer "F.Cu") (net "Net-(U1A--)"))
 (segment (start 111.725 105.65) (end 111.88 105.805) (width 1) (layer "F.Cu") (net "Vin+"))
 (segment (start 193.08 116.5) (end 193.08 116.77) (width 1) (layer "F.Cu") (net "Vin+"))
 (segment (start 192.85 116.5) (end 189.85 119.5) (width 1) (layer "F.Cu") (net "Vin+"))
 (segment (start 193.08 116.5) (end 192.85 116.5) (width 1) (layer "F.Cu") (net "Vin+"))
 (segment (start 105 105.65) (end 111.725 105.65) (width 1) (layer "F.Cu") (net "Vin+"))
 (segment (start 123.5 89.25) (end 124 88.75) (width 1) (layer "F.Cu") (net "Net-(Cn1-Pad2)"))
 (segment (start 105.15 68) (end 103 70.15) (width 1) (layer "F.Cu") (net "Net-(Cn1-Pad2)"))
 (segment (start 103 70.15) (end 103 87.75) (width 1) (layer "F.Cu") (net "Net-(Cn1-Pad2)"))
 (segment (start 103 87.75) (end 104.5 89.25) (width 1) (layer "F.Cu") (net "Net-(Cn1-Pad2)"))
 (segment (start 104.5 89.25) (end 123.5 89.25) (width 1) (layer "F.Cu") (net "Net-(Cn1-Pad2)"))
 (segment (start 112.1 118.35) (end 112.25 118.5) (width 1) (layer "F.Cu") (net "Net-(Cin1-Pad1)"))
 (segment (start 105 118.35) (end 112.1 118.35) (width 1) (layer "F.Cu") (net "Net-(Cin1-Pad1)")))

